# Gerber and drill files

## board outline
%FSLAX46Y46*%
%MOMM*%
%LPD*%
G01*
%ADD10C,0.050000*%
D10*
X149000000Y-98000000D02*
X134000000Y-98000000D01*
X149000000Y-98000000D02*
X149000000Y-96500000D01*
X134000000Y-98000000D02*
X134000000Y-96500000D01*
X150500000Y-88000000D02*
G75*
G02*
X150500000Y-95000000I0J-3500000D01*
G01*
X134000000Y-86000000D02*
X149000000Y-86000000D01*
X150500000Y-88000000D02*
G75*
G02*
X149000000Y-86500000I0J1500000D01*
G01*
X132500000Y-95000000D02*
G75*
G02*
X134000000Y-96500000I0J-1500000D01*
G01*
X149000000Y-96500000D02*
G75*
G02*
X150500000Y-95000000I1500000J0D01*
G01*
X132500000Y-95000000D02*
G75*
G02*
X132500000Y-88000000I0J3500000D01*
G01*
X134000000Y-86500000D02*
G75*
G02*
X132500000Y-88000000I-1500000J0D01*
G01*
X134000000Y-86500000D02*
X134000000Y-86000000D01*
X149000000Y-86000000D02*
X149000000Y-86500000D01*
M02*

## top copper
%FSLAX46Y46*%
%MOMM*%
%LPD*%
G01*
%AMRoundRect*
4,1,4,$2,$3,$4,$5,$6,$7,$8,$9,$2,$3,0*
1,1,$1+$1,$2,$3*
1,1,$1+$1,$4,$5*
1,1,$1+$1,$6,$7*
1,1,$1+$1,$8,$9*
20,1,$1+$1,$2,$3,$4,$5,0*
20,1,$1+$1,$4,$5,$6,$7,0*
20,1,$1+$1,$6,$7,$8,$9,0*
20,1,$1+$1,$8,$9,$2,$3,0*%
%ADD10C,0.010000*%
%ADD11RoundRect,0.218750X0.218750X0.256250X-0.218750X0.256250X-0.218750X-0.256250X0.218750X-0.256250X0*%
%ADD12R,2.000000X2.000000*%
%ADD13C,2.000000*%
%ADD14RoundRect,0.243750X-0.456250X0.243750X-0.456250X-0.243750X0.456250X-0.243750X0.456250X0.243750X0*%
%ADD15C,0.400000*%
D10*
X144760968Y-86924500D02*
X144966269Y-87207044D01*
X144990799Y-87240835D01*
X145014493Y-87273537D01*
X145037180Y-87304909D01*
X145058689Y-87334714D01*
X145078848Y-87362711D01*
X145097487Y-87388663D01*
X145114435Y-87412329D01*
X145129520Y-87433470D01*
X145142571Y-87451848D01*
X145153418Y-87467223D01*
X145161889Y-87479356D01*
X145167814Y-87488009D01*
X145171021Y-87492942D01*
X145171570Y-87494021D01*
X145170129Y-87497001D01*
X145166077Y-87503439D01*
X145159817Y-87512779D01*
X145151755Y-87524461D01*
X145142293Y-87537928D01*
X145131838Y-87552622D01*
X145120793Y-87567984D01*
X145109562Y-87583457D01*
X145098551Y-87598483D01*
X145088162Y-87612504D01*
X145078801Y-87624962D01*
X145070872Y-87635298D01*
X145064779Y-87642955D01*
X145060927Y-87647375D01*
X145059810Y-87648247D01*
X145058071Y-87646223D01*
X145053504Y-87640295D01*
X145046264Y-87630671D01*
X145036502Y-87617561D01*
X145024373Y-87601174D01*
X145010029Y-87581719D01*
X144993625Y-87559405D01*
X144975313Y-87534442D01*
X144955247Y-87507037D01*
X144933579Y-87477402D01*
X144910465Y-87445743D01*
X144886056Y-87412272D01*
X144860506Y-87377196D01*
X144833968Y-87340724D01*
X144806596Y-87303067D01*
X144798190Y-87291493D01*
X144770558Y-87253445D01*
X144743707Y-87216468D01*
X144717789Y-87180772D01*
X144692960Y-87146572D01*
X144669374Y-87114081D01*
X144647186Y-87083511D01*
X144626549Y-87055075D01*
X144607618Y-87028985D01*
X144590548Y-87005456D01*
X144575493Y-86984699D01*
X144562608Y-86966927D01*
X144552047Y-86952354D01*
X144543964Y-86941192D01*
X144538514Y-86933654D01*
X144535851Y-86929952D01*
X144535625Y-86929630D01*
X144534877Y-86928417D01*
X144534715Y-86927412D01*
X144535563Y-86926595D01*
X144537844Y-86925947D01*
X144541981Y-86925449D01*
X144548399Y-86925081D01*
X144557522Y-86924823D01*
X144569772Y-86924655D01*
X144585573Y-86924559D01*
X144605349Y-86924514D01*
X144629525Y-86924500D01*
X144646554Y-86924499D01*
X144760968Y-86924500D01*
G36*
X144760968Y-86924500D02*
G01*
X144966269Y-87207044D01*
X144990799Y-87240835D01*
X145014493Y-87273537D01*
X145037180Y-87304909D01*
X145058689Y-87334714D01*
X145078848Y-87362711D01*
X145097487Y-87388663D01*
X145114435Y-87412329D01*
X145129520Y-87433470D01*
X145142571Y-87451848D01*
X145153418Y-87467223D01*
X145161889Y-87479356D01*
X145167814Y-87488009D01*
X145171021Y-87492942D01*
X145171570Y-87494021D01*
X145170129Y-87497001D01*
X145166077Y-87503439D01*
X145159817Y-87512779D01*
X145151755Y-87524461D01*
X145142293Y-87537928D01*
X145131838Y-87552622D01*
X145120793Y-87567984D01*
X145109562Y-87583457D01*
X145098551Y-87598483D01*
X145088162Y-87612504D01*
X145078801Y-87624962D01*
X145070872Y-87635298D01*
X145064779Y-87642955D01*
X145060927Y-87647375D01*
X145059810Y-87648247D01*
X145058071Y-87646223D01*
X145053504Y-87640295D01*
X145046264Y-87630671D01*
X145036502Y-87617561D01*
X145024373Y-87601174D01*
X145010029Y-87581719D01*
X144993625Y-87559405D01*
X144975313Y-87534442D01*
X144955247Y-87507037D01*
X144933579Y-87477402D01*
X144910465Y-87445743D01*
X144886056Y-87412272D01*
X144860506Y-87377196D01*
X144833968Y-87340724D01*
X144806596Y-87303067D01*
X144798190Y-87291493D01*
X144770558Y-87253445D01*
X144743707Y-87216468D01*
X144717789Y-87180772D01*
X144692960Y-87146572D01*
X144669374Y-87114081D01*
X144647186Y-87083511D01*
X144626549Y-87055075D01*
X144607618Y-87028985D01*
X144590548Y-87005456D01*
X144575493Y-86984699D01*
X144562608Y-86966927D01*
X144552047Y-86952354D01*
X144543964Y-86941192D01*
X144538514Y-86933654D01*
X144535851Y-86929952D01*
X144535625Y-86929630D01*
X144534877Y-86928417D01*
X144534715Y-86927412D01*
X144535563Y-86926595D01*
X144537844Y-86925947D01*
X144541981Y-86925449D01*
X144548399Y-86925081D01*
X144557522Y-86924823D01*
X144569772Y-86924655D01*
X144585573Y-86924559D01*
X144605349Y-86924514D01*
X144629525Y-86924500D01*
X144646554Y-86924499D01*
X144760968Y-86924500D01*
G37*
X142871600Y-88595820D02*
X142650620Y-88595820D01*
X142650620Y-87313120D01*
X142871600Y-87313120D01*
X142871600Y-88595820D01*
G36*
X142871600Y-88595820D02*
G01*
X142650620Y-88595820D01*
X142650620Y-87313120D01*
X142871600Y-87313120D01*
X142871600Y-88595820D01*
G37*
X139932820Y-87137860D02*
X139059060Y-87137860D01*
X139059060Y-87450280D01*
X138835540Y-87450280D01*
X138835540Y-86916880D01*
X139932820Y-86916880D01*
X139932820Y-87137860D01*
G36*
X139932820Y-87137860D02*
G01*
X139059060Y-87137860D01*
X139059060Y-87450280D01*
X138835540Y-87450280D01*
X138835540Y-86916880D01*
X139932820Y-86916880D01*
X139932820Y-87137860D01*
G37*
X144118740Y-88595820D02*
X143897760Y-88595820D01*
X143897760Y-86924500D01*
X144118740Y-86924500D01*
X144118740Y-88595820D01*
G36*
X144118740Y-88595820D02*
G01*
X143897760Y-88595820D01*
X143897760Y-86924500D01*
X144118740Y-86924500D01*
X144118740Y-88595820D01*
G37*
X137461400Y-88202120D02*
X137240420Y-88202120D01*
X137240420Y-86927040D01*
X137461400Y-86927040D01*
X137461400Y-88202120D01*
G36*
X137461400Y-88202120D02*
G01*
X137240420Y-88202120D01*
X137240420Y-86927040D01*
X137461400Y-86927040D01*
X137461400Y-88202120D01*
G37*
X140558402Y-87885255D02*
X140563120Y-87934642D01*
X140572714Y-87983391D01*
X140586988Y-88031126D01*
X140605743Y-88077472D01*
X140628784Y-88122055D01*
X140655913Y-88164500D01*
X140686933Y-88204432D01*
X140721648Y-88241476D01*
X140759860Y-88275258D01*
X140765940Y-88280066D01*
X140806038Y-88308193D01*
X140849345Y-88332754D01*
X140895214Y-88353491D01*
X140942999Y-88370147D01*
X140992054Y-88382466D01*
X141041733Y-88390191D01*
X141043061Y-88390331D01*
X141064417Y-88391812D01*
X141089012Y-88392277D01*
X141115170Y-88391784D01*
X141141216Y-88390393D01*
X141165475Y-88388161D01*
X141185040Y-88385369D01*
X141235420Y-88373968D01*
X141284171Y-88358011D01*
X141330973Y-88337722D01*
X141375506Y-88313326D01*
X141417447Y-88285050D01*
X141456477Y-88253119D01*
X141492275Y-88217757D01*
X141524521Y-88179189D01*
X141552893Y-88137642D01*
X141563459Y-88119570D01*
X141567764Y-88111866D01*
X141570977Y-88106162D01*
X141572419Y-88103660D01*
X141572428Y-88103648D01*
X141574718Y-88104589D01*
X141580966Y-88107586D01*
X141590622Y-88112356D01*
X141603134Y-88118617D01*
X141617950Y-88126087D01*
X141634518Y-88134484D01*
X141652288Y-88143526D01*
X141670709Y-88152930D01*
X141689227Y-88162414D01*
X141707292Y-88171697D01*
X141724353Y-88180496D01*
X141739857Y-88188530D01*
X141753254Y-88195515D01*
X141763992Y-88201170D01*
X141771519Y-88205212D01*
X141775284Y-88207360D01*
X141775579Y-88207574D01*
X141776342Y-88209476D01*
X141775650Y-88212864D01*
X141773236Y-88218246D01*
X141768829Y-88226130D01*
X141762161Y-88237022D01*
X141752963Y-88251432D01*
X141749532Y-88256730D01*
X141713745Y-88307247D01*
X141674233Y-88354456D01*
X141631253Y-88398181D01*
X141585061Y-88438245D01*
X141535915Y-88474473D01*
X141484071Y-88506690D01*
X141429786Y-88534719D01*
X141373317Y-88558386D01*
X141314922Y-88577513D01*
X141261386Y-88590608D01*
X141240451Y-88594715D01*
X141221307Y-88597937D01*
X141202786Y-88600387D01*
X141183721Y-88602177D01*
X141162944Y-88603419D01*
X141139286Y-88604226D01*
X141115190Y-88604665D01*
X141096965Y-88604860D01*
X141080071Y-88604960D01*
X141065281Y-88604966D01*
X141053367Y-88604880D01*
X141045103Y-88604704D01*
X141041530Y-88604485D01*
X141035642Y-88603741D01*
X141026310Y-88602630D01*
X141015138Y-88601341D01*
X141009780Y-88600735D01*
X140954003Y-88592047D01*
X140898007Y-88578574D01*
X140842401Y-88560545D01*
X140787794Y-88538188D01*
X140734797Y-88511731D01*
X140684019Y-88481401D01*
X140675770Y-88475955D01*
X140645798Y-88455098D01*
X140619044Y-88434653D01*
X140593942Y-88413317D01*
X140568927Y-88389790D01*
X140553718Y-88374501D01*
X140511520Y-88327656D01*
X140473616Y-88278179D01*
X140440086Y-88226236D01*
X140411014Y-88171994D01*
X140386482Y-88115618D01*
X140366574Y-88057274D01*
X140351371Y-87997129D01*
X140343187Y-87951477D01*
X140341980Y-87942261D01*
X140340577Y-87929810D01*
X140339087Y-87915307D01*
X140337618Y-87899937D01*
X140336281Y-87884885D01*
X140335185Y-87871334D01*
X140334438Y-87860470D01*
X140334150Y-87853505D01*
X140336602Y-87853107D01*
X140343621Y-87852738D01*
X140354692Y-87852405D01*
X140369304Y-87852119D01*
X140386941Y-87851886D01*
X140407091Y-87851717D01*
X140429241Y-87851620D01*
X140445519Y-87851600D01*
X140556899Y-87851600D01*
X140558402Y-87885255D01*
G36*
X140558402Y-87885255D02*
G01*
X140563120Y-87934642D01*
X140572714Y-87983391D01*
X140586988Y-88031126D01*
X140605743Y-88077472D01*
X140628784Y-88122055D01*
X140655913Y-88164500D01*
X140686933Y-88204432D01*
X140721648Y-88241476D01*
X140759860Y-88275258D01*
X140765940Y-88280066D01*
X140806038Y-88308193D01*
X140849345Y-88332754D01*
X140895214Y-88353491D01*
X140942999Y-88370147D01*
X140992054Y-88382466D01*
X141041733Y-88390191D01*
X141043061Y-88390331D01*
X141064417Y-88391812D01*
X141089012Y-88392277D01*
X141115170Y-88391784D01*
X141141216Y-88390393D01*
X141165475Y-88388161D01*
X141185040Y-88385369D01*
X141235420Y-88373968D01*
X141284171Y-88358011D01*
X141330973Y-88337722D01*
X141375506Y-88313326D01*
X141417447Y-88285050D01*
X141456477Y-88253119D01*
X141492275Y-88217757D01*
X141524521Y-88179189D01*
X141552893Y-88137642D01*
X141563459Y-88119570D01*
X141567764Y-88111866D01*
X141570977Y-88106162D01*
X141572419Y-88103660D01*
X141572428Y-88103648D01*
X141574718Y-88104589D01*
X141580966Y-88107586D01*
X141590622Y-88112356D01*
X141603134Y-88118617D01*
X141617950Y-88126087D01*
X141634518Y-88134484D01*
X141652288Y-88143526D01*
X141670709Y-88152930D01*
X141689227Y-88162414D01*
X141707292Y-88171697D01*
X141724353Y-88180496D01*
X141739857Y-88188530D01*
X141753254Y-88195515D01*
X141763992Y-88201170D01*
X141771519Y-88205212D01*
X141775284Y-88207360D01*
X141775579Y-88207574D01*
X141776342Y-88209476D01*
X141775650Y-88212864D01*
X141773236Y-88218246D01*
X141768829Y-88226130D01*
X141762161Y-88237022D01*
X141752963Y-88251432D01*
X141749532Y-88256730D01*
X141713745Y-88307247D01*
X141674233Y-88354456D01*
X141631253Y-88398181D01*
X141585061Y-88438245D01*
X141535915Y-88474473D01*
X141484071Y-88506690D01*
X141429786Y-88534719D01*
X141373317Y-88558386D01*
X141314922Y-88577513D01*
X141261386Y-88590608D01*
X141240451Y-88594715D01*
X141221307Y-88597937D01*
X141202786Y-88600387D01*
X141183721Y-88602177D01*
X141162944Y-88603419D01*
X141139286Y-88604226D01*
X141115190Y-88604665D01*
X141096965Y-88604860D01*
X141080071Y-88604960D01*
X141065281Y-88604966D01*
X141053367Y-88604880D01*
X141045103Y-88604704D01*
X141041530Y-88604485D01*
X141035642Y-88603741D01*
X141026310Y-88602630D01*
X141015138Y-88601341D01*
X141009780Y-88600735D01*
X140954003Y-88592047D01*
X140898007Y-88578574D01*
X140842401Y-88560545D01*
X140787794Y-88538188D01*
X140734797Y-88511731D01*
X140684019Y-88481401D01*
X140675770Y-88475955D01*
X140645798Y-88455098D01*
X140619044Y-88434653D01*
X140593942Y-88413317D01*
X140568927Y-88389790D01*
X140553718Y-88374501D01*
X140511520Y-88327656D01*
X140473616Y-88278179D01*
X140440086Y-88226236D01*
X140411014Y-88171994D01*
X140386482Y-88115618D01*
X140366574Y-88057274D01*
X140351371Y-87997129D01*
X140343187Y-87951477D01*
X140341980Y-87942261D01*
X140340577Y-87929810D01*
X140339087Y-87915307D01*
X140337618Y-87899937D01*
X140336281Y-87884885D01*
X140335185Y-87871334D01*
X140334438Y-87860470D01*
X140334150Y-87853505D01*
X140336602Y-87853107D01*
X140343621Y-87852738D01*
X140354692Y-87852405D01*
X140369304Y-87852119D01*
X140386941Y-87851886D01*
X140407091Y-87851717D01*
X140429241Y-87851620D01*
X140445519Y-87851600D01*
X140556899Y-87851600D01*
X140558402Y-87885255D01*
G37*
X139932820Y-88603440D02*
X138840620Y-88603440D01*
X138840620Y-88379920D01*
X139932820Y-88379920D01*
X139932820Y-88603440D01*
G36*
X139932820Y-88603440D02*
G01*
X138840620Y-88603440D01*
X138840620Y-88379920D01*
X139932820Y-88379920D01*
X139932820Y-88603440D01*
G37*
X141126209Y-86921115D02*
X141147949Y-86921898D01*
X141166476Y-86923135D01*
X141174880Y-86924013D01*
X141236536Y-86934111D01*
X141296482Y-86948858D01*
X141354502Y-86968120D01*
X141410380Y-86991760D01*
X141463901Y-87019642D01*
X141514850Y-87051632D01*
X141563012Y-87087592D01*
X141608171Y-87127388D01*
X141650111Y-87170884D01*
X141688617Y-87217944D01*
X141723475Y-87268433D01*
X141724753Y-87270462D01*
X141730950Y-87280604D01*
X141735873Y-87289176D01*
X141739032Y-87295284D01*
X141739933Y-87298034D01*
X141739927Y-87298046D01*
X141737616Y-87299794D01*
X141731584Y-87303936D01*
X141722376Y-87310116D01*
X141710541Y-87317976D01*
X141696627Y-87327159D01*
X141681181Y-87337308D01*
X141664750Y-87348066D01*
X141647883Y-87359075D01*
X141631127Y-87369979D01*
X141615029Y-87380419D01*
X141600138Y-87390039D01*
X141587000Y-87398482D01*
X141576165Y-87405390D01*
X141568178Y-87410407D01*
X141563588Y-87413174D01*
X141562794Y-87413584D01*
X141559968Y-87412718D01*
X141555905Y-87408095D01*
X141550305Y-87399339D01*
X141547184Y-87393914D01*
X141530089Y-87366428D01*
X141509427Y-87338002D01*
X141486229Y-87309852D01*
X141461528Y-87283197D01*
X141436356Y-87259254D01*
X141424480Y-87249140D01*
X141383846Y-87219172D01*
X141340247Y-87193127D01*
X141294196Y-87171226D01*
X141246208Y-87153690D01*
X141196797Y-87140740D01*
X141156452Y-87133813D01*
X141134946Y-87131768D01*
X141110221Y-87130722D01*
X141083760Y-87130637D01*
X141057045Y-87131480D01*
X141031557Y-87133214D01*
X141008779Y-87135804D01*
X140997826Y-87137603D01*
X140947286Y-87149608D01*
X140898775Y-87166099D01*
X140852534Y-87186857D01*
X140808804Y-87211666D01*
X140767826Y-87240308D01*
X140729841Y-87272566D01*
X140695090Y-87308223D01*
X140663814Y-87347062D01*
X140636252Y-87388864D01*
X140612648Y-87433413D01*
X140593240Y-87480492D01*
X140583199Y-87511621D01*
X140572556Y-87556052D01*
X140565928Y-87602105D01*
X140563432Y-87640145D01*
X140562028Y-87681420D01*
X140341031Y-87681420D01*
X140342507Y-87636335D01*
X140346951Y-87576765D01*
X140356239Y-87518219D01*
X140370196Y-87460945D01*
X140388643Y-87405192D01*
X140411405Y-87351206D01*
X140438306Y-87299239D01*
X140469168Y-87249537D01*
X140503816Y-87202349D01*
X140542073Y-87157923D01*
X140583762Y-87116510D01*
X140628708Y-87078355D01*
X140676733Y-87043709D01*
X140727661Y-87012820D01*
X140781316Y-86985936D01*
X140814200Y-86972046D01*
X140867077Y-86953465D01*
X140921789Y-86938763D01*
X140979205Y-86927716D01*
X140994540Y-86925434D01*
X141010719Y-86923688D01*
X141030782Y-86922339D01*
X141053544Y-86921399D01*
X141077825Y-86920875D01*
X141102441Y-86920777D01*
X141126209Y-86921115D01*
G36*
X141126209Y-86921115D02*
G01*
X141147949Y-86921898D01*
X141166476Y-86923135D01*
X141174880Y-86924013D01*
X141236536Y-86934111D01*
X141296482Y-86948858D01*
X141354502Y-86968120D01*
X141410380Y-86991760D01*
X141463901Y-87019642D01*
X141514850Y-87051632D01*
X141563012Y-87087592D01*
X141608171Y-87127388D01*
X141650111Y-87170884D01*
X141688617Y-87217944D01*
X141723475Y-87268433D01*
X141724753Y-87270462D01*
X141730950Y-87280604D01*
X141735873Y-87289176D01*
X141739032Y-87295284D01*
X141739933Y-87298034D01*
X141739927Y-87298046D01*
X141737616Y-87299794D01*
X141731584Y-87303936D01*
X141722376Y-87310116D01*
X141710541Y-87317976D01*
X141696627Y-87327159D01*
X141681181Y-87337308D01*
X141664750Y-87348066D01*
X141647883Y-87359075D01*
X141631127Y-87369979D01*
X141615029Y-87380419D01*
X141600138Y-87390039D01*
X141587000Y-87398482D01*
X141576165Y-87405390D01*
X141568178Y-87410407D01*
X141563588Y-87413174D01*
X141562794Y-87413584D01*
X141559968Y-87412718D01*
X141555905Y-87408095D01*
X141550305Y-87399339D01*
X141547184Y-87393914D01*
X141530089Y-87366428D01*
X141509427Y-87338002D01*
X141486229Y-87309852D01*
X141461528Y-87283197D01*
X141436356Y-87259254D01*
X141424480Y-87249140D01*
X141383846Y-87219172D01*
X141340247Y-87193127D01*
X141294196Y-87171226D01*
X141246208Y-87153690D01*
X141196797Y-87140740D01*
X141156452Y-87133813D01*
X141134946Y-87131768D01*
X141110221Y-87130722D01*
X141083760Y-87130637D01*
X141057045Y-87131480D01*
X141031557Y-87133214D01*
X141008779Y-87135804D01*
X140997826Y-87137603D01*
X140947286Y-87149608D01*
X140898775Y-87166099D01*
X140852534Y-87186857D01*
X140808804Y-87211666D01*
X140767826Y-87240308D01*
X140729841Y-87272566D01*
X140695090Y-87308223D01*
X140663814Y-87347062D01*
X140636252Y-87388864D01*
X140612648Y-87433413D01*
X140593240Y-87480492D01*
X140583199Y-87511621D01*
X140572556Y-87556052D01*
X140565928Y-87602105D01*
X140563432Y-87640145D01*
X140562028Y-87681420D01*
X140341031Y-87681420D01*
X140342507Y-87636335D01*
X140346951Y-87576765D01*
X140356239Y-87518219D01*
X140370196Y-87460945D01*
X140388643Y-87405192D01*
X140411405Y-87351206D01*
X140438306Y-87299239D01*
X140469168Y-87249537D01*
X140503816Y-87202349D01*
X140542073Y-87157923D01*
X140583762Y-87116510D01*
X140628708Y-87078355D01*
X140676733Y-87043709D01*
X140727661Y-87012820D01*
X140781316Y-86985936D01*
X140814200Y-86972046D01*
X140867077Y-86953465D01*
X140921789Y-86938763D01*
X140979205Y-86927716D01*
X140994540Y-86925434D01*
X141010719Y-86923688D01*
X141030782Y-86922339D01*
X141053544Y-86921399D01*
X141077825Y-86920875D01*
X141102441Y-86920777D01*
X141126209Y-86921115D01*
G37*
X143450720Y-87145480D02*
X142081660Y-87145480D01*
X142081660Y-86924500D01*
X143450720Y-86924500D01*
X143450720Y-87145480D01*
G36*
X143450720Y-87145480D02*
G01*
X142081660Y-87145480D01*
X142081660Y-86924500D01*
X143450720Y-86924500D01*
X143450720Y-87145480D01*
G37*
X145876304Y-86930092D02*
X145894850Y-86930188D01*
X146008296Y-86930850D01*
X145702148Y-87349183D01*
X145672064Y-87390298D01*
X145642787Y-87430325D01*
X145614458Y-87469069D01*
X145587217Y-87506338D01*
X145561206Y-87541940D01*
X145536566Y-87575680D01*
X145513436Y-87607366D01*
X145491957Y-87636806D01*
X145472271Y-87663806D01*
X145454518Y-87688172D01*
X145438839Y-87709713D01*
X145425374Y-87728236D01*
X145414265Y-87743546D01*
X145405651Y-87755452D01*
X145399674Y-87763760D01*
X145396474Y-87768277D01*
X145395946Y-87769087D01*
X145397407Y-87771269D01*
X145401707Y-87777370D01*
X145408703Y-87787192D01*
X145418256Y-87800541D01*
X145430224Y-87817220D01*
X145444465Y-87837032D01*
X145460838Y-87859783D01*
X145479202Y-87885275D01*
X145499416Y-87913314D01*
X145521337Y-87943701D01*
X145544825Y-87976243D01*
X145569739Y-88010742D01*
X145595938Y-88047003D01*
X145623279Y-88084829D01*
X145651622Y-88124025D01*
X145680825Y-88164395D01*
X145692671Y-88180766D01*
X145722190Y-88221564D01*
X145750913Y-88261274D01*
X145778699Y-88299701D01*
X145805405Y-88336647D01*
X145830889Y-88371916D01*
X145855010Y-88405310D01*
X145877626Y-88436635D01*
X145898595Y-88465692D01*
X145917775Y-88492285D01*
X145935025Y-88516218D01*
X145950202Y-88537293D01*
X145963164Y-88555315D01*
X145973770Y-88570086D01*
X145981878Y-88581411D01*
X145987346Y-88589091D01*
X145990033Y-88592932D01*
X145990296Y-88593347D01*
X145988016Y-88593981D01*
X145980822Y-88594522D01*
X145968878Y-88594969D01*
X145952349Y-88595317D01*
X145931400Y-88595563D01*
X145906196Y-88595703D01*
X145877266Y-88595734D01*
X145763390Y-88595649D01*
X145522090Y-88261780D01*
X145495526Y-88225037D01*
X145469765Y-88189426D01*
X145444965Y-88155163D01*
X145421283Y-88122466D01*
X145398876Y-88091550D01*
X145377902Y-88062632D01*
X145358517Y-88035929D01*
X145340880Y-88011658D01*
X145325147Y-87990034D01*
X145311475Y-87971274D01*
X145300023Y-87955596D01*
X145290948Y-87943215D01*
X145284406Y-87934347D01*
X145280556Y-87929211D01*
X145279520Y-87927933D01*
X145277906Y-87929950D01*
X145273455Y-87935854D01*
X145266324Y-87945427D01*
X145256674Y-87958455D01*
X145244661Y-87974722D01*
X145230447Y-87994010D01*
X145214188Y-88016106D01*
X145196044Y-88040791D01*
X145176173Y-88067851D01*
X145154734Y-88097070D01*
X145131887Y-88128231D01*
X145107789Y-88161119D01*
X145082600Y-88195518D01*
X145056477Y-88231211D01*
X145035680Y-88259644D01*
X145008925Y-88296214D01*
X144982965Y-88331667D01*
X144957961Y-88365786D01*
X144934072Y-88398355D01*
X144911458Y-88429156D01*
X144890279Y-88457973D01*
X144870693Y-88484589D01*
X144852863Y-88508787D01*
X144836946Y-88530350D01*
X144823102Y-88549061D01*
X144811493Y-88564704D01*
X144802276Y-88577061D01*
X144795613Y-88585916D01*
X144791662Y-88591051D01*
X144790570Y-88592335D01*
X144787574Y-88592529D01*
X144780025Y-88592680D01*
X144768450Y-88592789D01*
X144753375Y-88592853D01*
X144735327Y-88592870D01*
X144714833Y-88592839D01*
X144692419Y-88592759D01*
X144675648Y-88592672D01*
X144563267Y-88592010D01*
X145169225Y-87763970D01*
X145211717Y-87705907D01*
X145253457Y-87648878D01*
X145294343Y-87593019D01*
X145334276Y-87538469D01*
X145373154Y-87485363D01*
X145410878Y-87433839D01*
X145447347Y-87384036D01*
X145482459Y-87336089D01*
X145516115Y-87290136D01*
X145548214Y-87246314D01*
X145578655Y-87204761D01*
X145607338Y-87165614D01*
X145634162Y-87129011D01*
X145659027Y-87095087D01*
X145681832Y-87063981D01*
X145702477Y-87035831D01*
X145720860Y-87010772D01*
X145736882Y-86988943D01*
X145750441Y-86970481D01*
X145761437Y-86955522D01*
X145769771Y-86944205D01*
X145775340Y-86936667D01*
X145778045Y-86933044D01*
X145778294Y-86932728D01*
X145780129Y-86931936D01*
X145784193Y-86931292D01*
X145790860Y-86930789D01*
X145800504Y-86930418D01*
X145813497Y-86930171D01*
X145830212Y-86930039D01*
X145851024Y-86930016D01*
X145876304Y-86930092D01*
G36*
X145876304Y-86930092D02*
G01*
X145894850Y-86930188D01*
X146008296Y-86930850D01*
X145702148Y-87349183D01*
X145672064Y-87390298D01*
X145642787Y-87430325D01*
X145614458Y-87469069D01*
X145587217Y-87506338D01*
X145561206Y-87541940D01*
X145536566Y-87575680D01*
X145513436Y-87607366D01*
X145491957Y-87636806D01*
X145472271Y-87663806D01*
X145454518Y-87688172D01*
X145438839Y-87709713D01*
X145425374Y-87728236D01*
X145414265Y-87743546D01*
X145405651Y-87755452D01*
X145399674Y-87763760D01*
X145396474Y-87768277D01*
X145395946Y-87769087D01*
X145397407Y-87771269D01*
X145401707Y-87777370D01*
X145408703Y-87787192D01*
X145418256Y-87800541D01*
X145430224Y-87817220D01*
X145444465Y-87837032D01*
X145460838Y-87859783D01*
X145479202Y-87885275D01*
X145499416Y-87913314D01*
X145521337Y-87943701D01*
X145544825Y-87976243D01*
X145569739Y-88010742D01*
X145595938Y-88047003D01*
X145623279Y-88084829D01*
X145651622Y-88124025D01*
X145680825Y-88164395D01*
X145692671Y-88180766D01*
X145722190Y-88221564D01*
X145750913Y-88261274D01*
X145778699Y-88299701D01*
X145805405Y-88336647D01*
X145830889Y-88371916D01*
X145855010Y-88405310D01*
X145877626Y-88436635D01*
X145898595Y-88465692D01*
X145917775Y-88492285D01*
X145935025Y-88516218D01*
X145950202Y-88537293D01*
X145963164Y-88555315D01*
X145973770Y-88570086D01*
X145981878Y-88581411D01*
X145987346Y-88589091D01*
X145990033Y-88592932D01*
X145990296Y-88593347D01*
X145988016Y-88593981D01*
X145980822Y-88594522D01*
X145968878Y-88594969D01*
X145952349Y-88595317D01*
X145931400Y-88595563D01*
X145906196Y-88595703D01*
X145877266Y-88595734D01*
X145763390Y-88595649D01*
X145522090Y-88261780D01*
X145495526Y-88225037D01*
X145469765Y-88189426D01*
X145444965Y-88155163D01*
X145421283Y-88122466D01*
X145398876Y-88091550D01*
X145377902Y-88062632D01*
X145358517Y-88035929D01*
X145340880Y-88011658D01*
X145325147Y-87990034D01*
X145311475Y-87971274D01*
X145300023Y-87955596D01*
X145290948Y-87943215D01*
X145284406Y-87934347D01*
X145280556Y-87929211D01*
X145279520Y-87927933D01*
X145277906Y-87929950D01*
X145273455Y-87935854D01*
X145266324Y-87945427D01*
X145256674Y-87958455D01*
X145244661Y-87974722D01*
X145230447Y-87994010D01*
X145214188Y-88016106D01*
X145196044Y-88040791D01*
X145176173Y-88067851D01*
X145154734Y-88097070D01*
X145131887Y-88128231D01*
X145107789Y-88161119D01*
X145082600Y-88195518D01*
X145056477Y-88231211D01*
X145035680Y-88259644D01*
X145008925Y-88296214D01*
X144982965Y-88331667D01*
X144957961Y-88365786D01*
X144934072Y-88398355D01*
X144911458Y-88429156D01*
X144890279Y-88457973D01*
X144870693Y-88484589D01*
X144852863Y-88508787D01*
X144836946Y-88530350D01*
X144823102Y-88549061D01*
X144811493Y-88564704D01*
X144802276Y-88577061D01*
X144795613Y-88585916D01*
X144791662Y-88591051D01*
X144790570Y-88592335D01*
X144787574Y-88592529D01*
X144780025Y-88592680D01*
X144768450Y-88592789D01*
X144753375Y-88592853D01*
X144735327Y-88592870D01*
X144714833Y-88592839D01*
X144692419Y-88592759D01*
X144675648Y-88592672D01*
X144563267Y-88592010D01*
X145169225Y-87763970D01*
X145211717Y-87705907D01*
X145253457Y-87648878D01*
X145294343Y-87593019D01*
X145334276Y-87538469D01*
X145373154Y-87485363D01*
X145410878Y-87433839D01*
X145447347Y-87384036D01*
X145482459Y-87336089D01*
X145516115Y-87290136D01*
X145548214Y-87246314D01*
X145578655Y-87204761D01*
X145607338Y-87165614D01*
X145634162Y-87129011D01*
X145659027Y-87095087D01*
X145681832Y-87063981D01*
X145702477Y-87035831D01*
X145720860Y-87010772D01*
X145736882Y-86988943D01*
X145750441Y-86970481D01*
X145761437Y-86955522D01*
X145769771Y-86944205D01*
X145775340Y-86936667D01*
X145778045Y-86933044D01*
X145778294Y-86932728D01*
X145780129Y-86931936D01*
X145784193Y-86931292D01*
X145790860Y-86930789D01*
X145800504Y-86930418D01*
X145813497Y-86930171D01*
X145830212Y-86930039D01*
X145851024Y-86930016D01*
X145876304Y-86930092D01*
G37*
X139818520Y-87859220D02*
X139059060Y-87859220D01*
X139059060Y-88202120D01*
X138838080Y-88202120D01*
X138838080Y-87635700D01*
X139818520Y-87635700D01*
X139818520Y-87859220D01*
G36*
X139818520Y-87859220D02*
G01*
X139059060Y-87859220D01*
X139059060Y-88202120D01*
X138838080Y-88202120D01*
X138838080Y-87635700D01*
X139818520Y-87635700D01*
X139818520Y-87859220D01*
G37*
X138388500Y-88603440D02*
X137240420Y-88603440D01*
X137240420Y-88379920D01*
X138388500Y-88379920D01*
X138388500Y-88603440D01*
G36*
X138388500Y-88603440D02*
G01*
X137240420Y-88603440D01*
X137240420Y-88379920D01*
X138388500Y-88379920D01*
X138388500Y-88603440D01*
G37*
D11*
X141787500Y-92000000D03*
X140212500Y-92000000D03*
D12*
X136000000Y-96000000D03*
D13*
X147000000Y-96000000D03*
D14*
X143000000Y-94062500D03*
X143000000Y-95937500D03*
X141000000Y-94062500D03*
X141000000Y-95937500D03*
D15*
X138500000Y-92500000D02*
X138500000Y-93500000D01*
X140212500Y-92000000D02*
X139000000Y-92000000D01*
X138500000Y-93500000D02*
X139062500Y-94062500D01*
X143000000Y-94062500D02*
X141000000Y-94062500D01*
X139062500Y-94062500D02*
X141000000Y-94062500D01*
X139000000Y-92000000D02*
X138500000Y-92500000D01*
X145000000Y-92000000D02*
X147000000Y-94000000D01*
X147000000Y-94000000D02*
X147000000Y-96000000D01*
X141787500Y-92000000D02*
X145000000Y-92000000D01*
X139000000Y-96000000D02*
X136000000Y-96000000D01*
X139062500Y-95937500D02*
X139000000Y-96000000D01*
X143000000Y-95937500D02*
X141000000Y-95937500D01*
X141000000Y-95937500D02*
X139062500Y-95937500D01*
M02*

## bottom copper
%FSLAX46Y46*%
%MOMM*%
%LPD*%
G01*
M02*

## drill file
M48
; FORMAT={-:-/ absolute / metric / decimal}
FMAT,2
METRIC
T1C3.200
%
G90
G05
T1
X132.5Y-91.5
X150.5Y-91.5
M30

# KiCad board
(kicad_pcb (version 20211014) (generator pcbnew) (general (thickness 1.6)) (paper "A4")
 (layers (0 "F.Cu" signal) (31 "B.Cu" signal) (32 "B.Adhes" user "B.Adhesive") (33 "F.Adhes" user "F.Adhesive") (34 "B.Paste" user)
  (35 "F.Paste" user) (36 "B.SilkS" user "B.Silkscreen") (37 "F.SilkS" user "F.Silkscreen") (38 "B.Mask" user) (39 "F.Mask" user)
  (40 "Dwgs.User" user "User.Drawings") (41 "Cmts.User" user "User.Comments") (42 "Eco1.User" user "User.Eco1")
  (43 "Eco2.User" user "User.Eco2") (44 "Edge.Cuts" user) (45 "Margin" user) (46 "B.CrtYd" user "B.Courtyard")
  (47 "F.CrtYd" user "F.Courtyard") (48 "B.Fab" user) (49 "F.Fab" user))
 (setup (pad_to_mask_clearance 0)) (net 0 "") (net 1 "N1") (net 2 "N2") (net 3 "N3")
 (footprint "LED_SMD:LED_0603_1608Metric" (layer "F.Cu") (at 141 92 180)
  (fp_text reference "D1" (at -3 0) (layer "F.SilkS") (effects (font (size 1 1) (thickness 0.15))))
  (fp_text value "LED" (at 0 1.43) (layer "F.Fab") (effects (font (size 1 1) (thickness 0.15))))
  (pad "1" smd roundrect locked (at -0.7875 0 180) (size 0.875 0.95) (layers "F.Cu" "F.Paste" "F.Mask") (roundrect_rratio 0.25) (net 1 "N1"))
  (pad "2" smd roundrect locked (at 0.7875 0 180) (size 0.875 0.95) (layers "F.Cu" "F.Paste" "F.Mask") (roundrect_rratio 0.25) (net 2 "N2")))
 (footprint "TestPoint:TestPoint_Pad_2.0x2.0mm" (layer "F.Cu") (at 136 96)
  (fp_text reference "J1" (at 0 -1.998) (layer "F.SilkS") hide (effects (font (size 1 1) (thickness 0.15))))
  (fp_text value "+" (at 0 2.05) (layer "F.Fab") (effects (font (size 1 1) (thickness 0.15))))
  (pad "1" smd rect locked (at 0 0) (size 2 2) (layers "F.Cu" "F.Mask") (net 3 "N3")))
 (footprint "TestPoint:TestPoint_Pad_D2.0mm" (layer "F.Cu") (at 147 96)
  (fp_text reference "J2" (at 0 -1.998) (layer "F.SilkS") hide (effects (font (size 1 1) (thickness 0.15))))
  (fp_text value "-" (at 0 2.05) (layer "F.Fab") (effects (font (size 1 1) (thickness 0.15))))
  (pad "1" smd circle locked (at 0 0) (size 2 2) (layers "F.Cu" "F.Mask") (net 1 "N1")))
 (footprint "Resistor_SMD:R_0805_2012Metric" (layer "F.Cu") (at 143 95 -90)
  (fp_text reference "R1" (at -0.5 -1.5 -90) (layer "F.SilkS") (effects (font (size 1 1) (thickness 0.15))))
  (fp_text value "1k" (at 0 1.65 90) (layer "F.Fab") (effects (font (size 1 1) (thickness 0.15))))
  (pad "1" smd roundrect locked (at -0.9375 0 270) (size 0.975 1.4) (layers "F.Cu" "F.Paste" "F.Mask") (roundrect_rratio 0.25) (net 2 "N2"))
  (pad "2" smd roundrect locked (at 0.9375 0 270) (size 0.975 1.4) (layers "F.Cu" "F.Paste" "F.Mask") (roundrect_rratio 0.25) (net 3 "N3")))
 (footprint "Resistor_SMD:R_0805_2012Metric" (layer "F.Cu") (at 141 95 -90)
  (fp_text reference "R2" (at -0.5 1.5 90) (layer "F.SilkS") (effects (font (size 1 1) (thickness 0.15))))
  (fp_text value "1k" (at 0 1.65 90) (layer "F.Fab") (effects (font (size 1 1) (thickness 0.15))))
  (pad "1" smd roundrect locked (at -0.9375 0 270) (size 0.975 1.4) (layers "F.Cu" "F.Paste" "F.Mask") (roundrect_rratio 0.25) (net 2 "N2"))
  (pad "2" smd roundrect locked (at 0.9375 0 270) (size 0.975 1.4) (layers "F.Cu" "F.Paste" "F.Mask") (roundrect_rratio 0.25) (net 3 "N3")))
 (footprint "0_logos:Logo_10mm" (layer "F.Cu") (at 141.5 87.75)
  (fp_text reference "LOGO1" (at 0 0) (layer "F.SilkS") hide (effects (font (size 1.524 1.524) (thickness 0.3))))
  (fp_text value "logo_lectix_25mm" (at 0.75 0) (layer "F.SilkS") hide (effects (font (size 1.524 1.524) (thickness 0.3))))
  (fp_poly
   (pts (xy 3.260968 -0.8255) (xy 3.466269 -0.542956) (xy 3.490799 -0.509165) (xy 3.514493 -0.476463) (xy 3.53718 -0.445091)
    (xy 3.558689 -0.415286) (xy 3.578848 -0.387289) (xy 3.597487 -0.361337) (xy 3.614435 -0.337671) (xy 3.62952 -0.31653)
    (xy 3.642571 -0.298152) (xy 3.653418 -0.282777) (xy 3.661889 -0.270644) (xy 3.667814 -0.261991) (xy 3.671021 -0.257058)
    (xy 3.67157 -0.255979) (xy 3.670129 -0.252999) (xy 3.666077 -0.246561) (xy 3.659817 -0.237221) (xy 3.651755 -0.225539)
    (xy 3.642293 -0.212072) (xy 3.631838 -0.197378) (xy 3.620793 -0.182016) (xy 3.609562 -0.166543) (xy 3.598551 -0.151517)
    (xy 3.588162 -0.137496) (xy 3.578801 -0.125038) (xy 3.570872 -0.114702) (xy 3.564779 -0.107045) (xy 3.560927 -0.102625)
    (xy 3.55981 -0.101753) (xy 3.558071 -0.103777) (xy 3.553504 -0.109705) (xy 3.546264 -0.119329) (xy 3.536502 -0.132439)
    (xy 3.524373 -0.148826) (xy 3.510029 -0.168281) (xy 3.493625 -0.190595) (xy 3.475313 -0.215558) (xy 3.455247 -0.242963)
    (xy 3.433579 -0.272598) (xy 3.410465 -0.304257) (xy 3.386056 -0.337728) (xy 3.360506 -0.372804) (xy 3.333968 -0.409276)
    (xy 3.306596 -0.446933) (xy 3.29819 -0.458507) (xy 3.270558 -0.496555) (xy 3.243707 -0.533532) (xy 3.217789 -0.569228)
    (xy 3.19296 -0.603428) (xy 3.169374 -0.635919) (xy 3.147186 -0.666489) (xy 3.126549 -0.694925) (xy 3.107618 -0.721015)
    (xy 3.090548 -0.744544) (xy 3.075493 -0.765301) (xy 3.062608 -0.783073) (xy 3.052047 -0.797646) (xy 3.043964 -0.808808)
    (xy 3.038514 -0.816346) (xy 3.035851 -0.820048) (xy 3.035625 -0.82037) (xy 3.034877 -0.821583) (xy 3.034715 -0.822588)
    (xy 3.035563 -0.823405) (xy 3.037844 -0.824053) (xy 3.041981 -0.824551) (xy 3.048399 -0.824919) (xy 3.057522 -0.825177)
    (xy 3.069772 -0.825345) (xy 3.085573 -0.825441) (xy 3.105349 -0.825486) (xy 3.129525 -0.8255) (xy 3.146554 -0.825501)
    (xy 3.260968 -0.8255))
   (layer "F.Cu") (width 0.01) (fill solid))
  (fp_poly
   (pts (xy 1.3716 0.84582) (xy 1.15062 0.84582) (xy 1.15062 -0.43688) (xy 1.3716 -0.43688) (xy 1.3716 0.84582)) (layer "F.Cu") (width 0.01)
   (fill solid))
  (fp_poly
   (pts (xy -1.56718 -0.61214) (xy -2.44094 -0.61214) (xy -2.44094 -0.29972) (xy -2.66446 -0.29972) (xy -2.66446 -0.83312)
    (xy -1.56718 -0.83312) (xy -1.56718 -0.61214))
   (layer "F.Cu") (width 0.01) (fill solid))
  (fp_poly
   (pts (xy 2.61874 0.84582) (xy 2.39776 0.84582) (xy 2.39776 -0.8255) (xy 2.61874 -0.8255) (xy 2.61874 0.84582)) (layer "F.Cu")
   (width 0.01) (fill solid))
  (fp_poly
   (pts (xy -4.0386 0.45212) (xy -4.25958 0.45212) (xy -4.25958 -0.82296) (xy -4.0386 -0.82296) (xy -4.0386 0.45212)) (layer "F.Cu")
   (width 0.01) (fill solid))
  (fp_poly
   (pts (xy -0.941598 0.135255) (xy -0.93688 0.184642) (xy -0.927286 0.233391) (xy -0.913012 0.281126) (xy -0.894257 0.327472)
    (xy -0.871216 0.372055) (xy -0.844087 0.4145) (xy -0.813067 0.454432) (xy -0.778352 0.491476) (xy -0.74014 0.525258)
    (xy -0.73406 0.530066) (xy -0.693962 0.558193) (xy -0.650655 0.582754) (xy -0.604786 0.603491) (xy -0.557001 0.620147)
    (xy -0.507946 0.632466) (xy -0.458267 0.640191) (xy -0.456939 0.640331) (xy -0.435583 0.641812) (xy -0.410988 0.642277)
    (xy -0.38483 0.641784) (xy -0.358784 0.640393) (xy -0.334525 0.638161) (xy -0.31496 0.635369) (xy -0.26458 0.623968)
    (xy -0.215829 0.608011) (xy -0.169027 0.587722) (xy -0.124494 0.563326) (xy -0.082553 0.53505) (xy -0.043523 0.503119)
    (xy -0.007725 0.467757) (xy 0.024521 0.429189) (xy 0.052893 0.387642) (xy 0.063459 0.36957) (xy 0.067764 0.361866)
    (xy 0.070977 0.356162) (xy 0.072419 0.35366) (xy 0.072428 0.353648) (xy 0.074718 0.354589) (xy 0.080966 0.357586) (xy 0.090622 0.362356)
    (xy 0.103134 0.368617) (xy 0.11795 0.376087) (xy 0.134518 0.384484) (xy 0.152288 0.393526) (xy 0.170709 0.40293) (xy 0.189227 0.412414)
    (xy 0.207292 0.421697) (xy 0.224353 0.430496) (xy 0.239857 0.43853) (xy 0.253254 0.445515) (xy 0.263992 0.45117) (xy 0.271519 0.455212)
    (xy 0.275284 0.45736) (xy 0.275579 0.457574) (xy 0.276342 0.459476) (xy 0.27565 0.462864) (xy 0.273236 0.468246) (xy 0.268829 0.47613)
    (xy 0.262161 0.487022) (xy 0.252963 0.501432) (xy 0.249532 0.50673) (xy 0.213745 0.557247) (xy 0.174233 0.604456) (xy 0.131253 0.648181)
    (xy 0.085061 0.688245) (xy 0.035915 0.724473) (xy -0.015929 0.75669) (xy -0.070214 0.784719) (xy -0.126683 0.808386)
    (xy -0.185078 0.827513) (xy -0.238614 0.840608) (xy -0.259549 0.844715) (xy -0.278693 0.847937) (xy -0.297214 0.850387)
    (xy -0.316279 0.852177) (xy -0.337056 0.853419) (xy -0.360714 0.854226) (xy -0.38481 0.854665) (xy -0.403035 0.85486)
    (xy -0.419929 0.85496) (xy -0.434719 0.854966) (xy -0.446633 0.85488) (xy -0.454897 0.854704) (xy -0.45847 0.854485)
    (xy -0.464358 0.853741) (xy -0.47369 0.85263) (xy -0.484862 0.851341) (xy -0.49022 0.850735) (xy -0.545997 0.842047)
    (xy -0.601993 0.828574) (xy -0.657599 0.810545) (xy -0.712206 0.788188) (xy -0.765203 0.761731) (xy -0.815981 0.731401)
    (xy -0.82423 0.725955) (xy -0.854202 0.705098) (xy -0.880956 0.684653) (xy -0.906058 0.663317) (xy -0.931073 0.63979)
    (xy -0.946282 0.624501) (xy -0.98848 0.577656) (xy -1.026384 0.528179) (xy -1.059914 0.476236) (xy -1.088986 0.421994)
    (xy -1.113518 0.365618) (xy -1.133426 0.307274) (xy -1.148629 0.247129) (xy -1.156813 0.201477) (xy -1.15802 0.192261)
    (xy -1.159423 0.17981) (xy -1.160913 0.165307) (xy -1.162382 0.149937) (xy -1.163719 0.134885) (xy -1.164815 0.121334)
    (xy -1.165562 0.11047) (xy -1.16585 0.103505) (xy -1.163398 0.103107) (xy -1.156379 0.102738) (xy -1.145308 0.102405)
    (xy -1.130696 0.102119) (xy -1.113059 0.101886) (xy -1.092909 0.101717) (xy -1.070759 0.10162) (xy -1.054481 0.1016)
    (xy -0.943101 0.1016) (xy -0.941598 0.135255))
   (layer "F.Cu") (width 0.01) (fill solid))
  (fp_poly
   (pts (xy -1.56718 0.85344) (xy -2.65938 0.85344) (xy -2.65938 0.62992) (xy -1.56718 0.62992) (xy -1.56718 0.85344)) (layer "F.Cu")
   (width 0.01) (fill solid))
  (fp_poly
   (pts (xy -0.373791 -0.828885) (xy -0.352051 -0.828102) (xy -0.333524 -0.826865) (xy -0.32512 -0.825987) (xy -0.263464 -0.815889)
    (xy -0.203518 -0.801142) (xy -0.145498 -0.78188) (xy -0.08962 -0.75824) (xy -0.036099 -0.730358) (xy 0.01485 -0.698368)
    (xy 0.063012 -0.662408) (xy 0.108171 -0.622612) (xy 0.150111 -0.579116) (xy 0.188617 -0.532056) (xy 0.223475 -0.481567)
    (xy 0.224753 -0.479538) (xy 0.23095 -0.469396) (xy 0.235873 -0.460824) (xy 0.239032 -0.454716) (xy 0.239933 -0.451966)
    (xy 0.239927 -0.451954) (xy 0.237616 -0.450206) (xy 0.231584 -0.446064) (xy 0.222376 -0.439884) (xy 0.210541 -0.432024)
    (xy 0.196627 -0.422841) (xy 0.181181 -0.412692) (xy 0.16475 -0.401934) (xy 0.147883 -0.390925) (xy 0.131127 -0.380021)
    (xy 0.115029 -0.369581) (xy 0.100138 -0.359961) (xy 0.087 -0.351518) (xy 0.076165 -0.34461) (xy 0.068178 -0.339593)
    (xy 0.063588 -0.336826) (xy 0.062794 -0.336416) (xy 0.059968 -0.337282) (xy 0.055905 -0.341905) (xy 0.050305 -0.350661)
    (xy 0.047184 -0.356086) (xy 0.030089 -0.383572) (xy 0.009427 -0.411998) (xy -0.013771 -0.440148) (xy -0.038472 -0.466803)
    (xy -0.063644 -0.490746) (xy -0.07552 -0.50086) (xy -0.116154 -0.530828) (xy -0.159753 -0.556873) (xy -0.205804 -0.578774)
    (xy -0.253792 -0.59631) (xy -0.303203 -0.60926) (xy -0.343548 -0.616187) (xy -0.365054 -0.618232) (xy -0.389779 -0.619278)
    (xy -0.41624 -0.619363) (xy -0.442955 -0.61852) (xy -0.468443 -0.616786) (xy -0.491221 -0.614196) (xy -0.502174 -0.612397)
    (xy -0.552714 -0.600392) (xy -0.601225 -0.583901) (xy -0.647466 -0.563143) (xy -0.691196 -0.538334) (xy -0.732174 -0.509692)
    (xy -0.770159 -0.477434) (xy -0.80491 -0.441777) (xy -0.836186 -0.402938) (xy -0.863748 -0.361136) (xy -0.887352 -0.316587)
    (xy -0.90676 -0.269508) (xy -0.916801 -0.238379) (xy -0.927444 -0.193948) (xy -0.934072 -0.147895) (xy -0.936568 -0.109855)
    (xy -0.937972 -0.06858) (xy -1.158969 -0.06858) (xy -1.157493 -0.113665) (xy -1.153049 -0.173235) (xy -1.143761 -0.231781)
    (xy -1.129804 -0.289055) (xy -1.111357 -0.344808) (xy -1.088595 -0.398794) (xy -1.061694 -0.450761) (xy -1.030832 -0.500463)
    (xy -0.996184 -0.547651) (xy -0.957927 -0.592077) (xy -0.916238 -0.63349) (xy -0.871292 -0.671645) (xy -0.823267 -0.706291)
    (xy -0.772339 -0.73718) (xy -0.718684 -0.764064) (xy -0.6858 -0.777954) (xy -0.632923 -0.796535) (xy -0.578211 -0.811237)
    (xy -0.520795 -0.822284) (xy -0.50546 -0.824566) (xy -0.489281 -0.826312) (xy -0.469218 -0.827661) (xy -0.446456 -0.828601)
    (xy -0.422175 -0.829125) (xy -0.397559 -0.829223) (xy -0.373791 -0.828885))
   (layer "F.Cu") (width 0.01) (fill solid))
  (fp_poly
   (pts (xy 1.95072 -0.60452) (xy 0.58166 -0.60452) (xy 0.58166 -0.8255) (xy 1.95072 -0.8255) (xy 1.95072 -0.60452)) (layer "F.Cu")
   (width 0.01) (fill solid))
  (fp_poly
   (pts (xy 4.376304 -0.819908) (xy 4.39485 -0.819812) (xy 4.508296 -0.81915) (xy 4.202148 -0.400817) (xy 4.172064 -0.359702)
    (xy 4.142787 -0.319675) (xy 4.114458 -0.280931) (xy 4.087217 -0.243662) (xy 4.061206 -0.20806) (xy 4.036566 -0.17432)
    (xy 4.013436 -0.142634) (xy 3.991957 -0.113194) (xy 3.972271 -0.086194) (xy 3.954518 -0.061828) (xy 3.938839 -0.040287)
    (xy 3.925374 -0.021764) (xy 3.914265 -0.006454) (xy 3.905651 0.005452) (xy 3.899674 0.01376) (xy 3.896474 0.018277)
    (xy 3.895946 0.019087) (xy 3.897407 0.021269) (xy 3.901707 0.02737) (xy 3.908703 0.037192) (xy 3.918256 0.050541) (xy 3.930224 0.06722)
    (xy 3.944465 0.087032) (xy 3.960838 0.109783) (xy 3.979202 0.135275) (xy 3.999416 0.163314) (xy 4.021337 0.193701)
    (xy 4.044825 0.226243) (xy 4.069739 0.260742) (xy 4.095938 0.297003) (xy 4.123279 0.334829) (xy 4.151622 0.374025)
    (xy 4.180825 0.414395) (xy 4.192671 0.430766) (xy 4.22219 0.471564) (xy 4.250913 0.511274) (xy 4.278699 0.549701) (xy 4.305405 0.586647)
    (xy 4.330889 0.621916) (xy 4.35501 0.65531) (xy 4.377626 0.686635) (xy 4.398595 0.715692) (xy 4.417775 0.742285) (xy 4.435025 0.766218)
    (xy 4.450202 0.787293) (xy 4.463164 0.805315) (xy 4.47377 0.820086) (xy 4.481878 0.831411) (xy 4.487346 0.839091) (xy 4.490033 0.842932)
    (xy 4.490296 0.843347) (xy 4.488016 0.843981) (xy 4.480822 0.844522) (xy 4.468878 0.844969) (xy 4.452349 0.845317) (xy 4.4314 0.845563)
    (xy 4.406196 0.845703) (xy 4.377266 0.845734) (xy 4.26339 0.845649) (xy 4.02209 0.51178) (xy 3.995526 0.475037) (xy 3.969765 0.439426)
    (xy 3.944965 0.405163) (xy 3.921283 0.372466) (xy 3.898876 0.34155) (xy 3.877902 0.312632) (xy 3.858517 0.285929) (xy 3.84088 0.261658)
    (xy 3.825147 0.240034) (xy 3.811475 0.221274) (xy 3.800023 0.205596) (xy 3.790948 0.193215) (xy 3.784406 0.184347)
    (xy 3.780556 0.179211) (xy 3.77952 0.177933) (xy 3.777906 0.17995) (xy 3.773455 0.185854) (xy 3.766324 0.195427) (xy 3.756674 0.208455)
    (xy 3.744661 0.224722) (xy 3.730447 0.24401) (xy 3.714188 0.266106) (xy 3.696044 0.290791) (xy 3.676173 0.317851) (xy 3.654734 0.34707)
    (xy 3.631887 0.378231) (xy 3.607789 0.411119) (xy 3.5826 0.445518) (xy 3.556477 0.481211) (xy 3.53568 0.509644) (xy 3.508925 0.546214)
    (xy 3.482965 0.581667) (xy 3.457961 0.615786) (xy 3.434072 0.648355) (xy 3.411458 0.679156) (xy 3.390279 0.707973)
    (xy 3.370693 0.734589) (xy 3.352863 0.758787) (xy 3.336946 0.78035) (xy 3.323102 0.799061) (xy 3.311493 0.814704) (xy 3.302276 0.827061)
    (xy 3.295613 0.835916) (xy 3.291662 0.841051) (xy 3.29057 0.842335) (xy 3.287574 0.842529) (xy 3.280025 0.84268) (xy 3.26845 0.842789)
    (xy 3.253375 0.842853) (xy 3.235327 0.84287) (xy 3.214833 0.842839) (xy 3.192419 0.842759) (xy 3.175648 0.842672) (xy 3.063267 0.84201)
    (xy 3.669225 0.01397) (xy 3.711717 -0.044093) (xy 3.753457 -0.101122) (xy 3.794343 -0.156981) (xy 3.834276 -0.211531)
    (xy 3.873154 -0.264637) (xy 3.910878 -0.316161) (xy 3.947347 -0.365964) (xy 3.982459 -0.413911) (xy 4.016115 -0.459864)
    (xy 4.048214 -0.503686) (xy 4.078655 -0.545239) (xy 4.107338 -0.584386) (xy 4.134162 -0.620989) (xy 4.159027 -0.654913)
    (xy 4.181832 -0.686019) (xy 4.202477 -0.714169) (xy 4.22086 -0.739228) (xy 4.236882 -0.761057) (xy 4.250441 -0.779519)
    (xy 4.261437 -0.794478) (xy 4.269771 -0.805795) (xy 4.27534 -0.813333) (xy 4.278045 -0.816956) (xy 4.278294 -0.817272)
    (xy 4.280129 -0.818064) (xy 4.284193 -0.818708) (xy 4.29086 -0.819211) (xy 4.300504 -0.819582) (xy 4.313497 -0.819829)
    (xy 4.330212 -0.819961) (xy 4.351024 -0.819984) (xy 4.376304 -0.819908))
   (layer "F.Cu") (width 0.01) (fill solid))
  (fp_poly
   (pts (xy -1.68148 0.10922) (xy -2.44094 0.10922) (xy -2.44094 0.45212) (xy -2.66192 0.45212) (xy -2.66192 -0.1143) (xy -1.68148 -0.1143)
    (xy -1.68148 0.10922))
   (layer "F.Cu") (width 0.01) (fill solid))
  (fp_poly
   (pts (xy -3.1115 0.85344) (xy -4.25958 0.85344) (xy -4.25958 0.62992) (xy -3.1115 0.62992) (xy -3.1115 0.85344)) (layer "F.Cu")
   (width 0.01) (fill solid)))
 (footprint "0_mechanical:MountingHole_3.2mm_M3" (layer "F.Cu") (at 132.5 91.5)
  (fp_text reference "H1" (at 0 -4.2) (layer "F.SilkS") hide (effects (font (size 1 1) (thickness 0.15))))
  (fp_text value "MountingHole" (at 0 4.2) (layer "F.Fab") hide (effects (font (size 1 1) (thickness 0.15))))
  (pad "" np_thru_hole circle locked (at 0 0) (size 3.2 3.2) (drill 3.2) (layers *.Cu *.Mask)))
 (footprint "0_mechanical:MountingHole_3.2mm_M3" (layer "F.Cu") (at 150.5 91.5)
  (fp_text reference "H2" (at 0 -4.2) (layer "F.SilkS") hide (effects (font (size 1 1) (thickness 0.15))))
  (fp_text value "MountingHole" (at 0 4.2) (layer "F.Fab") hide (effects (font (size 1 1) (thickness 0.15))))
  (pad "" np_thru_hole circle locked (at 0 0) (size 3.2 3.2) (drill 3.2) (layers *.Cu *.Mask)))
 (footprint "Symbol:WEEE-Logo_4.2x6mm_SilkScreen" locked (layer "B.Cu") (at 141.5 92 180)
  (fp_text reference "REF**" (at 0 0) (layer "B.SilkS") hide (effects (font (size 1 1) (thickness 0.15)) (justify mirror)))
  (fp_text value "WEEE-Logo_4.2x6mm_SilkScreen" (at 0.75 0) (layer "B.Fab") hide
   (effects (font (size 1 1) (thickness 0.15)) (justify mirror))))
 (gr_line (start 149 98) (end 134 98) (layer "Edge.Cuts") (width 0.05))
 (gr_line (start 149 98) (end 149 96.5) (layer "Edge.Cuts") (width 0.05))
 (gr_line (start 134 98) (end 134 96.5) (layer "Edge.Cuts") (width 0.05))
 (gr_arc (start 150.5 88) (mid 154 91.5) (end 150.5 95) (layer "Edge.Cuts") (width 0.05))
 (gr_line (start 134 86) (end 149 86) (layer "Edge.Cuts") (width 0.05))
 (gr_arc (start 150.5 88) (mid 149.43934 87.56066) (end 149 86.5) (layer "Edge.Cuts") (width 0.05))
 (gr_arc (start 132.5 95) (mid 133.56066 95.43934) (end 134 96.5) (layer "Edge.Cuts") (width 0.05))
 (gr_arc (start 149 96.5) (mid 149.43934 95.43934) (end 150.5 95) (layer "Edge.Cuts") (width 0.05))
 (gr_arc (start 132.5 95) (mid 129 91.5) (end 132.5 88) (layer "Edge.Cuts") (width 0.05))
 (gr_arc (start 134 86.5) (mid 133.56066 87.56066) (end 132.5 88) (layer "Edge.Cuts") (width 0.05))
 (gr_line (start 134 86.5) (end 134 86) (layer "Edge.Cuts") (width 0.05))
 (gr_line (start 149 86) (end 149 86.5) (layer "Edge.Cuts") (width 0.05))
 (segment (start 138.5 92.5) (end 138.5 93.5) (width 0.4) (layer "F.Cu") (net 2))
 (segment (start 140.2125 92) (end 139 92) (width 0.4) (layer "F.Cu") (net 2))
 (segment (start 138.5 93.5) (end 139.0625 94.0625) (width 0.4) (layer "F.Cu") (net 2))
 (segment (start 143 94.0625) (end 141 94.0625) (width 0.4) (layer "F.Cu") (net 2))
 (segment (start 139.0625 94.0625) (end 141 94.0625) (width 0.4) (layer "F.Cu") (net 2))
 (segment (start 139 92) (end 138.5 92.5) (width 0.4) (layer "F.Cu") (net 2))
 (segment (start 145 92) (end 147 94) (width 0.4) (layer "F.Cu") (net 1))
 (segment (start 147 94) (end 147 96) (width 0.4) (layer "F.Cu") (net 1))
 (segment (start 141.7875 92) (end 145 92) (width 0.4) (layer "F.Cu") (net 1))
 (segment (start 139 96) (end 136 96) (width 0.4) (layer "F.Cu") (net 3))
 (segment (start 139.0625 95.9375) (end 139 96) (width 0.4) (layer "F.Cu") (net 3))
 (segment (start 143 95.9375) (end 141 95.9375) (width 0.4) (layer "F.Cu") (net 3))
 (segment (start 141 95.9375) (end 139.0625 95.9375) (width 0.4) (layer "F.Cu") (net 3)))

